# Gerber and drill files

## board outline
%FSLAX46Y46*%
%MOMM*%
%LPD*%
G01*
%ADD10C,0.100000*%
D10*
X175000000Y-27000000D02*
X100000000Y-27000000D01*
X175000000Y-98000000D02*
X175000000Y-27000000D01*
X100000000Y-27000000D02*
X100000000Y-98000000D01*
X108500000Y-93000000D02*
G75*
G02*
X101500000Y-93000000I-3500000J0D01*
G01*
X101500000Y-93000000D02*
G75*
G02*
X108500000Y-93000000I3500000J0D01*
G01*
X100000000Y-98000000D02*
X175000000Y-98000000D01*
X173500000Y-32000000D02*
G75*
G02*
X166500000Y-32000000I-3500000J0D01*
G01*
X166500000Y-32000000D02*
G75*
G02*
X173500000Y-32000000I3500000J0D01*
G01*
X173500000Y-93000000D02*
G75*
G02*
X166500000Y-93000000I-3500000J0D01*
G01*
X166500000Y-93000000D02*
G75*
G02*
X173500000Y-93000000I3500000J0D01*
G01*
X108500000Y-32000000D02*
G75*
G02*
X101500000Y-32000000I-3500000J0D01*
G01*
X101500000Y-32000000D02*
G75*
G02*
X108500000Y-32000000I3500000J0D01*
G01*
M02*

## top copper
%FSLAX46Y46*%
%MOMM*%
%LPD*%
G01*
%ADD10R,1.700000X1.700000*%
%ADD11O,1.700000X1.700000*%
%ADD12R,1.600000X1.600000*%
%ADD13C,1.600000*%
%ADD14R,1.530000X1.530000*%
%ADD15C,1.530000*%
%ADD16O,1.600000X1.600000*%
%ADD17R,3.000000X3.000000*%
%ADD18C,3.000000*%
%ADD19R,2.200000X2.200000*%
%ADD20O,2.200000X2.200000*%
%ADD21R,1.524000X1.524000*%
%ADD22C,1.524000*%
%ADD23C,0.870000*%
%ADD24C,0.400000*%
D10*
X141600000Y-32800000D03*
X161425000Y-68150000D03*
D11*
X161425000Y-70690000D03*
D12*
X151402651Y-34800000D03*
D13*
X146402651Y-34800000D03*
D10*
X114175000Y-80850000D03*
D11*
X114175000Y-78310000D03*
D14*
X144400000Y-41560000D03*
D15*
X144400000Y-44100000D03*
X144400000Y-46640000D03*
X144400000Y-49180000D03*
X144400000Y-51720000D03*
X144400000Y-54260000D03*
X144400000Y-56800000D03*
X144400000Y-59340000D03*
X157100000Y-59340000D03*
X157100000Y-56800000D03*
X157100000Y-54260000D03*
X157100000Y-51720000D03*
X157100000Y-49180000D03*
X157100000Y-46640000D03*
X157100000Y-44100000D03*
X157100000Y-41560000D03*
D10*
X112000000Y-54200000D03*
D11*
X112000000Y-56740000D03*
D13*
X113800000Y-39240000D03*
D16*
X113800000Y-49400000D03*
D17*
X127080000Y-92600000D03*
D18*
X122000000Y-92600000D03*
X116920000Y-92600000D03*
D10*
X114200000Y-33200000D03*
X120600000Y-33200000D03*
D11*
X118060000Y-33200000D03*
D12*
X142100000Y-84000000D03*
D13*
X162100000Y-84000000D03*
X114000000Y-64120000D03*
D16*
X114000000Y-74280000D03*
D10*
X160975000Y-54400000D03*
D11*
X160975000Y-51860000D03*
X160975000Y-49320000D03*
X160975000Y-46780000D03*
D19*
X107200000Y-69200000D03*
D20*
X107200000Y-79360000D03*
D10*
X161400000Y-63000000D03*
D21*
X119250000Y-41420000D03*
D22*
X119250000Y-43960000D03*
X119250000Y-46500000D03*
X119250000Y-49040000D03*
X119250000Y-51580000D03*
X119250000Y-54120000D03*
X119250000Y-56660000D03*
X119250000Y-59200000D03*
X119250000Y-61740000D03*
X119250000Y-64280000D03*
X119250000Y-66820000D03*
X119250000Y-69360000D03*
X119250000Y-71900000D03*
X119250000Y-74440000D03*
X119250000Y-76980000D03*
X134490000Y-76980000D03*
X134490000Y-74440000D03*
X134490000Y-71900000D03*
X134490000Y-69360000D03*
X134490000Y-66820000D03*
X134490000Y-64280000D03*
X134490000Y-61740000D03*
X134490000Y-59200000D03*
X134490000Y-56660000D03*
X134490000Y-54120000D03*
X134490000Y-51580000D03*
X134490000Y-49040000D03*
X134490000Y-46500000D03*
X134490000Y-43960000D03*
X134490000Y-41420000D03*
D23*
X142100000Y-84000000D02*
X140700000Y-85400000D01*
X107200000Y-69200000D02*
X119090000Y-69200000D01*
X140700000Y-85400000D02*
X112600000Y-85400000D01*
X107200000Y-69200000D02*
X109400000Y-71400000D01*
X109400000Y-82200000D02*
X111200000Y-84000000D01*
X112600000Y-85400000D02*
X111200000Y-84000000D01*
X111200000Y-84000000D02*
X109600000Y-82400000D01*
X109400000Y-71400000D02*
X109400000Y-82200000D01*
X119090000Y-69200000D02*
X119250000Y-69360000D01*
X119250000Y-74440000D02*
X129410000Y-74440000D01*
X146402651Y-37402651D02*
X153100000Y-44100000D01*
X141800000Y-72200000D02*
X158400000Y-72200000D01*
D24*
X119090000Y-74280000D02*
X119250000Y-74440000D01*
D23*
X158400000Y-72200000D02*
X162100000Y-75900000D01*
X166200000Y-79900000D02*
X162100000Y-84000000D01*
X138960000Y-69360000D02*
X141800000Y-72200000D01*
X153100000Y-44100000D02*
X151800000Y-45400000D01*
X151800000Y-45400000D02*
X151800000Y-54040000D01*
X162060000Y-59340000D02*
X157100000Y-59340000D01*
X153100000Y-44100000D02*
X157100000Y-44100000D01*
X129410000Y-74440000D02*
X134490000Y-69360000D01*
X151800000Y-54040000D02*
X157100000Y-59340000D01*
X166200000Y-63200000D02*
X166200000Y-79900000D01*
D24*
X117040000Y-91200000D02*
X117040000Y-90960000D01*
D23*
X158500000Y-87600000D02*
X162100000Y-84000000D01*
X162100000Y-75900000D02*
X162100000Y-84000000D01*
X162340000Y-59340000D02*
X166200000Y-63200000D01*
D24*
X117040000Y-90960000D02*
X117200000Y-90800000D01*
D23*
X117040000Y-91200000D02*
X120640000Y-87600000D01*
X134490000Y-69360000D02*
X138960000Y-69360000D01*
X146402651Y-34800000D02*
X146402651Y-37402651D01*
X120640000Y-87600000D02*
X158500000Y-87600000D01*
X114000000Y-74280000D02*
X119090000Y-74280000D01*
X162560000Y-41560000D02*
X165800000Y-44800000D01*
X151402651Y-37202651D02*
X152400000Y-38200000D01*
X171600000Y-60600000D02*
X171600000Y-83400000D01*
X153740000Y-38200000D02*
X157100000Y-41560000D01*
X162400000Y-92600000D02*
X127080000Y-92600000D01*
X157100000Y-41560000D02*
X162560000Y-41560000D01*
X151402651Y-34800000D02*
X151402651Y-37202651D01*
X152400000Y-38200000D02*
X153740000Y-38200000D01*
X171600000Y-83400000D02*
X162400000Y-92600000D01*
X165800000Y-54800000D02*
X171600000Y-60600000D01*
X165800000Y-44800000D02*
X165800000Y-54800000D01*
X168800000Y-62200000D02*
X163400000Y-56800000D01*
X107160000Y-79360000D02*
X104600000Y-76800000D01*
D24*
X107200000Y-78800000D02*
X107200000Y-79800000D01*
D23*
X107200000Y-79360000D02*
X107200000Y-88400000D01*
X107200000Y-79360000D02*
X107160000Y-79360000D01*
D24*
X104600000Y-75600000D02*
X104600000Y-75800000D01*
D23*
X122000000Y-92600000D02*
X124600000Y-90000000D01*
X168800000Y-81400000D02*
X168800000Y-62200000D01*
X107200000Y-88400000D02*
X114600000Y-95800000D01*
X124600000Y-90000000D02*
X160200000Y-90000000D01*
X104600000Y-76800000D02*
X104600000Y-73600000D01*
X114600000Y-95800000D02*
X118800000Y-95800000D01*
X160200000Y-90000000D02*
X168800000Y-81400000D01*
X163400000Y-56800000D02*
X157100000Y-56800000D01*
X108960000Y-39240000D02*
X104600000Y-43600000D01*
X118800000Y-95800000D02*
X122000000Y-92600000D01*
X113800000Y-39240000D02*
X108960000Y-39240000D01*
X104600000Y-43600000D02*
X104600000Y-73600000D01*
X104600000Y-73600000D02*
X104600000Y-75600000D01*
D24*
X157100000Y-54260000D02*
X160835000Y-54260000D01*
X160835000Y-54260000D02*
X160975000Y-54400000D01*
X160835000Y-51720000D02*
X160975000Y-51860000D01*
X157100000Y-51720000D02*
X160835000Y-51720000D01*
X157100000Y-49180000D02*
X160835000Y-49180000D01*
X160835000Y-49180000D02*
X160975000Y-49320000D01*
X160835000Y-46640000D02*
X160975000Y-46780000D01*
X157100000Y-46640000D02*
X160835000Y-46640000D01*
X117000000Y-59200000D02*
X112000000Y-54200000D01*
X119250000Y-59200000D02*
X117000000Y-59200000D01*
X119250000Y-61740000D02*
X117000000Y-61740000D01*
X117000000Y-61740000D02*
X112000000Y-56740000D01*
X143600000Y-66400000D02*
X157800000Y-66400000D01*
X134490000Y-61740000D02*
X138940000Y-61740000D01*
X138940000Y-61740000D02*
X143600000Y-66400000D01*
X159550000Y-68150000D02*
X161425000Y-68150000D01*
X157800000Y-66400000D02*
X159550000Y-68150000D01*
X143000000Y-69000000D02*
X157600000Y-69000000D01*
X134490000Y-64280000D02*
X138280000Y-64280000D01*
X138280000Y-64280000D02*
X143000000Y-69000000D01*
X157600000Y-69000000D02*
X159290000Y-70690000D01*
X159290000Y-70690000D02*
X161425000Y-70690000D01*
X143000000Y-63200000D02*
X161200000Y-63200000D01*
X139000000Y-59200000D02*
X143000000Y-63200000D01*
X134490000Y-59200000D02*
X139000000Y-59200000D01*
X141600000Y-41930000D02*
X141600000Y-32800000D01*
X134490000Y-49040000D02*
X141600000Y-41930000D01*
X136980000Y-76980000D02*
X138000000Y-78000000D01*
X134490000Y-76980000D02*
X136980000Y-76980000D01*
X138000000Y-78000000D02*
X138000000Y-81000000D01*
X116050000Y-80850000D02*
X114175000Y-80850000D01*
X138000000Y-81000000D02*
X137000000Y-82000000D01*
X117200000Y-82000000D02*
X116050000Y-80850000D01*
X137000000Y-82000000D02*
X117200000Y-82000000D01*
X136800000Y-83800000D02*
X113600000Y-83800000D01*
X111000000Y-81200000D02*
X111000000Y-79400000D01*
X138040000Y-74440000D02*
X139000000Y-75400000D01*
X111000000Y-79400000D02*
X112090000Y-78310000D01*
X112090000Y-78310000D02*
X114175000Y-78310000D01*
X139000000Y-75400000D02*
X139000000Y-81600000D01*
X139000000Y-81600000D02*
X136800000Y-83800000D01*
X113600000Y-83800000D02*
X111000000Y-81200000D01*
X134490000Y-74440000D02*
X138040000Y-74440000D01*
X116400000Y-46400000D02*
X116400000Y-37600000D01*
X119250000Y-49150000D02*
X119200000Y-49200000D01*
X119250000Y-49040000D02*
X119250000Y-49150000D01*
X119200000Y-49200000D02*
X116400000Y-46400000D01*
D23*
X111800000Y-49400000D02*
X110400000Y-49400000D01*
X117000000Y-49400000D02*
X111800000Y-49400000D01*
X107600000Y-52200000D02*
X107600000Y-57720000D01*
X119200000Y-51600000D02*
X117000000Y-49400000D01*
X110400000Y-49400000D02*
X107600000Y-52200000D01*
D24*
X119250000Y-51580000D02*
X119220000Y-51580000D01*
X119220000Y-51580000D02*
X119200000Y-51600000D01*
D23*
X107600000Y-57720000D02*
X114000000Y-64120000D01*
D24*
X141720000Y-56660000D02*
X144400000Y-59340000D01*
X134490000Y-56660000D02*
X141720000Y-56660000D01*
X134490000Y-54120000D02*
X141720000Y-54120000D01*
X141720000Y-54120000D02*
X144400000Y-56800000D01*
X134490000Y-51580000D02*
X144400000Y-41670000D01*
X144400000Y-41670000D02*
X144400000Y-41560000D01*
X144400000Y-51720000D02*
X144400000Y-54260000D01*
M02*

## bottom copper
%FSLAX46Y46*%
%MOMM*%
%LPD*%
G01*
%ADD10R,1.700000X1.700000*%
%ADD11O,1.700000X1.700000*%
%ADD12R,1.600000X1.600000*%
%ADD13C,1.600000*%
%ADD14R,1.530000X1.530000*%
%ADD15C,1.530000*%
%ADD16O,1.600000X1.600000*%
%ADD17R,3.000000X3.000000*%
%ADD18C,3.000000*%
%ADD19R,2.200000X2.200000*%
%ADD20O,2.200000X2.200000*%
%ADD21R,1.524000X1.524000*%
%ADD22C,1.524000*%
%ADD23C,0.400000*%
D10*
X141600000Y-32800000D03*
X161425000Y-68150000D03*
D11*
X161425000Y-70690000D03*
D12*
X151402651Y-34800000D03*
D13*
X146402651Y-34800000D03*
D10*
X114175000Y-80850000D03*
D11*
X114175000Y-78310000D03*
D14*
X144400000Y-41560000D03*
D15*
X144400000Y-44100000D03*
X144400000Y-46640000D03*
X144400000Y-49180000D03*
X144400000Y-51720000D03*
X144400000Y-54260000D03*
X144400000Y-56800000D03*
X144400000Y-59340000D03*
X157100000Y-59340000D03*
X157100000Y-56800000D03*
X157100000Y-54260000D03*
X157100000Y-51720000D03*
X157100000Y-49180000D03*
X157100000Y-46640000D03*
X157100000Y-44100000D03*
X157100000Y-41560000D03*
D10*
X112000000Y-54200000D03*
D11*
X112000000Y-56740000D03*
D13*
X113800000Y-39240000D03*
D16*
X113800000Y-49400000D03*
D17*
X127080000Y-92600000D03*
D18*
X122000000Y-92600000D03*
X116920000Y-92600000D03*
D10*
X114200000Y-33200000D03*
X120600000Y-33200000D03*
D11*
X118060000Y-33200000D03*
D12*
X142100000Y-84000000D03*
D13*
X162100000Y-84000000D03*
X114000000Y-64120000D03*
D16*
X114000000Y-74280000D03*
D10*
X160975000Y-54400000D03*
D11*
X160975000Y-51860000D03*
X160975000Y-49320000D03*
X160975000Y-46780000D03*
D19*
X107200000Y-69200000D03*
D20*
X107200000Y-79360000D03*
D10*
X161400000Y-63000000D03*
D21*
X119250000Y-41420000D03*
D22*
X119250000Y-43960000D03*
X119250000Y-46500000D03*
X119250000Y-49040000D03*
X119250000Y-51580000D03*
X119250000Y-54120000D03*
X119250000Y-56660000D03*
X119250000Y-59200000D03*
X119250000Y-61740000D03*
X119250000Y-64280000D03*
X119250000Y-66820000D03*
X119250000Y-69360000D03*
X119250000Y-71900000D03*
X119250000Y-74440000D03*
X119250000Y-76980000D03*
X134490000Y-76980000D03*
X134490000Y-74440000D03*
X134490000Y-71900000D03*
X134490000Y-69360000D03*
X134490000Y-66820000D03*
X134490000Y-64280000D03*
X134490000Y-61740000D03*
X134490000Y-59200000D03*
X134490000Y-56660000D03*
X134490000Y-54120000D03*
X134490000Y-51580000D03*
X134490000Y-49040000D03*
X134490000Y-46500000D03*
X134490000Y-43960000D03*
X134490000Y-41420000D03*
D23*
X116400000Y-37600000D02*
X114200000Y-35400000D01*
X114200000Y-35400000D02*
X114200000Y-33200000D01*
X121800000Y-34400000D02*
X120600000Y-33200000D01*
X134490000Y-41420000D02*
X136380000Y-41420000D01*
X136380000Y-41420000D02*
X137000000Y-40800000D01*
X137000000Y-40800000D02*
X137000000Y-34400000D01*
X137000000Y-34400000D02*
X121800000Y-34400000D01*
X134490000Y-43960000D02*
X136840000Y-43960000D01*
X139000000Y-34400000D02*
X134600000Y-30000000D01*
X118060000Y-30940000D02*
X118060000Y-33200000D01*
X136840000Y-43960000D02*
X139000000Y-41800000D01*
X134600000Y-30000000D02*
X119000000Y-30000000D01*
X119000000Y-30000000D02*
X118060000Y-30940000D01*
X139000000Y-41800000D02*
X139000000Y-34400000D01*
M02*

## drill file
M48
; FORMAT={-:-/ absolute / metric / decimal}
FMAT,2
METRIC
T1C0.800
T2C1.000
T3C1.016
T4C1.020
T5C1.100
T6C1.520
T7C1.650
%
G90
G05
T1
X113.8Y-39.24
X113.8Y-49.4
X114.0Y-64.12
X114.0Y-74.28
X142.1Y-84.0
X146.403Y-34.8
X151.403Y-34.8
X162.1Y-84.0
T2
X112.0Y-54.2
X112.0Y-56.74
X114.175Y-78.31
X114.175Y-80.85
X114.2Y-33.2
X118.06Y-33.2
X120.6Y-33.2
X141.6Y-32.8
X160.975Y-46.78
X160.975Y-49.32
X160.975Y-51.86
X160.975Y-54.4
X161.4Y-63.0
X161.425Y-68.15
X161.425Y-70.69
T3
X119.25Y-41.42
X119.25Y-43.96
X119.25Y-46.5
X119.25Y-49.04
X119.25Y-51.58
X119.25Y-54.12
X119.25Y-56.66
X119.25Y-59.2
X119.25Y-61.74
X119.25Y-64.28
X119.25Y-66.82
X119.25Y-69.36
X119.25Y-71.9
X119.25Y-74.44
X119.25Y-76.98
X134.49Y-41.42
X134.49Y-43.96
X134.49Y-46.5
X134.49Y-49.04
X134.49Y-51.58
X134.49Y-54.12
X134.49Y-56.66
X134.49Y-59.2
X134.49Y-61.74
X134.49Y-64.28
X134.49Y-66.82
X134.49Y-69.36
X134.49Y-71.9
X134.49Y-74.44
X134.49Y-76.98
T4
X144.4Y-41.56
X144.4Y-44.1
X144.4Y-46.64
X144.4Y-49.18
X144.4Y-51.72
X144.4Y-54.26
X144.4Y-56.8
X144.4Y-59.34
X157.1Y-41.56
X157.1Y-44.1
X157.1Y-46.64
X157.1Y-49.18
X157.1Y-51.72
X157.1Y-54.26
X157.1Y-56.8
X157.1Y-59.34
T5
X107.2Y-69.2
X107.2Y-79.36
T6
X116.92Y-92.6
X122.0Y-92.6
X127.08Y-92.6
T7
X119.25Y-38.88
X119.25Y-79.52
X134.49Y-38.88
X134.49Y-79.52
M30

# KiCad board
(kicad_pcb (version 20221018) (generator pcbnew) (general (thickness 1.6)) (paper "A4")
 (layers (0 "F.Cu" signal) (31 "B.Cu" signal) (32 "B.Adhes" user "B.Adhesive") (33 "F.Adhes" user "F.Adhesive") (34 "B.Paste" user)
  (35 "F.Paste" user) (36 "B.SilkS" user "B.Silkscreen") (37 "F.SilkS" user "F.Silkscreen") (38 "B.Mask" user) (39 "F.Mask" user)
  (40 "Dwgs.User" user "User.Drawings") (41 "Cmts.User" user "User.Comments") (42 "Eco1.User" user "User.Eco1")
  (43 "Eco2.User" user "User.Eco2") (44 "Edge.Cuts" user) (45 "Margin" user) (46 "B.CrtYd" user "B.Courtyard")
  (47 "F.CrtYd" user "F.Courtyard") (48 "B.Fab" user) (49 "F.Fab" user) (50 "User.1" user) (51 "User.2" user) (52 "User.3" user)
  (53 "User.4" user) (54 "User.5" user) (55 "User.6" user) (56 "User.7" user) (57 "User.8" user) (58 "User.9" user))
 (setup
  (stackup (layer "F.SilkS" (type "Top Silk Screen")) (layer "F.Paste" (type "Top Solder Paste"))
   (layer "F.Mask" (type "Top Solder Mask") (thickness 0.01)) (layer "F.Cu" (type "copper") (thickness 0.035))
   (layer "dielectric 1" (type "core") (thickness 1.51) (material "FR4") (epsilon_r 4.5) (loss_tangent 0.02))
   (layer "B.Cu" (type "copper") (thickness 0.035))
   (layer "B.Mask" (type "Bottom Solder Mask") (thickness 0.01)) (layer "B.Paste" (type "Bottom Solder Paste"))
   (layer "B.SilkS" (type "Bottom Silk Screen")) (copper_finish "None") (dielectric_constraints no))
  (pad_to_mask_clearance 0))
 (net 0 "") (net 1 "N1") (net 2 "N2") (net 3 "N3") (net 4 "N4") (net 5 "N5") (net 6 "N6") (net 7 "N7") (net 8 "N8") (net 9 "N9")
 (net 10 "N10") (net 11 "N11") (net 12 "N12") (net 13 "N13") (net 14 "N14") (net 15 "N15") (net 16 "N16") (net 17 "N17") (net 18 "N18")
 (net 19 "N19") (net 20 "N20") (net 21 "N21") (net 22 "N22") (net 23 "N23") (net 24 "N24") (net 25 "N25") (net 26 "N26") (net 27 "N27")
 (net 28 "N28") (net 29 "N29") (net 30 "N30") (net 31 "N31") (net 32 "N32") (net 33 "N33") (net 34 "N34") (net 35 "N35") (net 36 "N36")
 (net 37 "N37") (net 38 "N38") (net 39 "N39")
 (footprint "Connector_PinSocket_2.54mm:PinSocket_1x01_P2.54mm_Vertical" (layer "F.Cu") (at 141.6 32.8)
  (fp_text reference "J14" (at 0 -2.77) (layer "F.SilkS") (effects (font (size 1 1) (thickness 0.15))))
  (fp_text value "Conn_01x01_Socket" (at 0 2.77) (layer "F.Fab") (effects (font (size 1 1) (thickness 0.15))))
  (pad "1" thru_hole rect (at 0 0) (size 1.7 1.7) (drill 1) (layers "*.Cu" "*.Mask") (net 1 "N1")))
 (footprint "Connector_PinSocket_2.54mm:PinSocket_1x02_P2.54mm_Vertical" (layer "F.Cu") (at 161.425 68.15)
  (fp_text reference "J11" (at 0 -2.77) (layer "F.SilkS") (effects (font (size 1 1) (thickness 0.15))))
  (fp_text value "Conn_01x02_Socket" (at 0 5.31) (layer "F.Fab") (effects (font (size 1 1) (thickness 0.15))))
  (pad "1" thru_hole rect (at 0 0) (size 1.7 1.7) (drill 1) (layers "*.Cu" "*.Mask") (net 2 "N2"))
  (pad "2" thru_hole oval (at 0 2.54) (size 1.7 1.7) (drill 1) (layers "*.Cu" "*.Mask") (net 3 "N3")))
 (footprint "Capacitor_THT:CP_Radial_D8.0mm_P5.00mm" (layer "F.Cu") (at 151.402651 34.8 180)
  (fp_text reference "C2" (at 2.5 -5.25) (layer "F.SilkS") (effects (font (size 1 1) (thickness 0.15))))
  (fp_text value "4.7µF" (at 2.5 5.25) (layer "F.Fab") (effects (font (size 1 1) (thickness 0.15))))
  (pad "1" thru_hole rect (at 0 0 180) (size 1.6 1.6) (drill 0.8) (layers "*.Cu" "*.Mask") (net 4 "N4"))
  (pad "2" thru_hole circle (at 5 0 180) (size 1.6 1.6) (drill 0.8) (layers "*.Cu" "*.Mask") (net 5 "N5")))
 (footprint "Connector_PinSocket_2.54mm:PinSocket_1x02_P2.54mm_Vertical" (layer "F.Cu") (at 114.175 80.85 180)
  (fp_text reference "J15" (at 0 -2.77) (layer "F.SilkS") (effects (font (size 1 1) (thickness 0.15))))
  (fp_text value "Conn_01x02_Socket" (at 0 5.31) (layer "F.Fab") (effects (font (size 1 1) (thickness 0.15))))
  (pad "1" thru_hole rect (at 0 0 180) (size 1.7 1.7) (drill 1) (layers "*.Cu" "*.Mask") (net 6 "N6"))
  (pad "2" thru_hole oval (at 0 2.54 180) (size 1.7 1.7) (drill 1) (layers "*.Cu" "*.Mask") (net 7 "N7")))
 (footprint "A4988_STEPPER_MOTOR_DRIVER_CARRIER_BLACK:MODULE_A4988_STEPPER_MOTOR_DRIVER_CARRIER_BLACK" (layer "F.Cu") (at 150.75 50.45)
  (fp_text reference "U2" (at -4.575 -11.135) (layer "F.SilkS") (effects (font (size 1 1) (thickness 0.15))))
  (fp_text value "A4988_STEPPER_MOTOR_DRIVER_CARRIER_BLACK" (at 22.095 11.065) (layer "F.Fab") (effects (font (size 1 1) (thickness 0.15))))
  (pad "1" thru_hole rect (at -6.35 -8.89) (size 1.53 1.53) (drill 1.02) (layers "*.Cu" "*.Mask") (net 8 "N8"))
  (pad "2" thru_hole circle (at -6.35 -6.35) (size 1.53 1.53) (drill 1.02) (layers "*.Cu" "*.Mask") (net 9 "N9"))
  (pad "3" thru_hole circle (at -6.35 -3.81) (size 1.53 1.53) (drill 1.02) (layers "*.Cu" "*.Mask") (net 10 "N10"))
  (pad "4" thru_hole circle (at -6.35 -1.27) (size 1.53 1.53) (drill 1.02) (layers "*.Cu" "*.Mask") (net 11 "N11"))
  (pad "5" thru_hole circle (at -6.35 1.27) (size 1.53 1.53) (drill 1.02) (layers "*.Cu" "*.Mask") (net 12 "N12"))
  (pad "6" thru_hole circle (at -6.35 3.81) (size 1.53 1.53) (drill 1.02) (layers "*.Cu" "*.Mask") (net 12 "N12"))
  (pad "7" thru_hole circle (at -6.35 6.35) (size 1.53 1.53) (drill 1.02) (layers "*.Cu" "*.Mask") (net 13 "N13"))
  (pad "8" thru_hole circle (at -6.35 8.89) (size 1.53 1.53) (drill 1.02) (layers "*.Cu" "*.Mask") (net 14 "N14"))
  (pad "9" thru_hole circle (at 6.35 8.89) (size 1.53 1.53) (drill 1.02) (layers "*.Cu" "*.Mask") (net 5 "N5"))
  (pad "10" thru_hole circle (at 6.35 6.35) (size 1.53 1.53) (drill 1.02) (layers "*.Cu" "*.Mask") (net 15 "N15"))
  (pad "11" thru_hole circle (at 6.35 3.81) (size 1.53 1.53) (drill 1.02) (layers "*.Cu" "*.Mask") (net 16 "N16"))
  (pad "12" thru_hole circle (at 6.35 1.27) (size 1.53 1.53) (drill 1.02) (layers "*.Cu" "*.Mask") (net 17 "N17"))
  (pad "13" thru_hole circle (at 6.35 -1.27) (size 1.53 1.53) (drill 1.02) (layers "*.Cu" "*.Mask") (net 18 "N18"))
  (pad "14" thru_hole circle (at 6.35 -3.81) (size 1.53 1.53) (drill 1.02) (layers "*.Cu" "*.Mask") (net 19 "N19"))
  (pad "15" thru_hole circle (at 6.35 -6.35) (size 1.53 1.53) (drill 1.02) (layers "*.Cu" "*.Mask") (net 5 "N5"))
  (pad "16" thru_hole circle (at 6.35 -8.89) (size 1.53 1.53) (drill 1.02) (layers "*.Cu" "*.Mask") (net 4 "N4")))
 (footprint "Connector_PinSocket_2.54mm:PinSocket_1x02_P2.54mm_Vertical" (layer "F.Cu") (at 112 54.2)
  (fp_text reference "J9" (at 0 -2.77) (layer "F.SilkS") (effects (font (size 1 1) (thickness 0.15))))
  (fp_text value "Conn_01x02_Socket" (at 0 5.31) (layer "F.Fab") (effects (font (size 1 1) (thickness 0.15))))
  (pad "1" thru_hole rect (at 0 0) (size 1.7 1.7) (drill 1) (layers "*.Cu" "*.Mask") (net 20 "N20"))
  (pad "2" thru_hole oval (at 0 2.54) (size 1.7 1.7) (drill 1) (layers "*.Cu" "*.Mask") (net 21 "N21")))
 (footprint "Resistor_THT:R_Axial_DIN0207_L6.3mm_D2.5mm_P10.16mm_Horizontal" (layer "F.Cu") (at 113.8 39.24 -90)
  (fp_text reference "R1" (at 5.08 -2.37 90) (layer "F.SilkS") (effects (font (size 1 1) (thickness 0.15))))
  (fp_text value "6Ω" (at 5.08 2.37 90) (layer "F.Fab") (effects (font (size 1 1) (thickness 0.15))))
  (pad "1" thru_hole circle (at 0 0 270) (size 1.6 1.6) (drill 0.8) (layers "*.Cu" "*.Mask") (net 15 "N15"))
  (pad "2" thru_hole oval (at 10.16 0 270) (size 1.6 1.6) (drill 0.8) (layers "*.Cu" "*.Mask") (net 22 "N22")))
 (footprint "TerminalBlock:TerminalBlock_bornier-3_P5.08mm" (layer "F.Cu") (at 127.08 92.6 180)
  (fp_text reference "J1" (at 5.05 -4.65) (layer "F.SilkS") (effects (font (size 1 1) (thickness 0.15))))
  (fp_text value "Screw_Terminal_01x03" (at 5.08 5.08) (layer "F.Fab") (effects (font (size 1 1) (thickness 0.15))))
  (pad "1" thru_hole rect (at 0 0 180) (size 3 3) (drill 1.52) (layers "*.Cu" "*.Mask") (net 4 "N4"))
  (pad "2" thru_hole circle (at 5.08 0 180) (size 3 3) (drill 1.52) (layers "*.Cu" "*.Mask") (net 15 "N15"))
  (pad "3" thru_hole circle (at 10.16 0 180) (size 3 3) (drill 1.52) (layers "*.Cu" "*.Mask") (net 5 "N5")))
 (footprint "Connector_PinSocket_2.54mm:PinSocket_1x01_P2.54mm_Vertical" (layer "F.Cu") (at 114.2 33.2)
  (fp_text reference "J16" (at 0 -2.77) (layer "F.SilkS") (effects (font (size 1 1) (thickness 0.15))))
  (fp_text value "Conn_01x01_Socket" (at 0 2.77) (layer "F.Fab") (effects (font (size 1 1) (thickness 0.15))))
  (pad "1" thru_hole rect (at 0 0) (size 1.7 1.7) (drill 1) (layers "*.Cu" "*.Mask") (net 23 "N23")))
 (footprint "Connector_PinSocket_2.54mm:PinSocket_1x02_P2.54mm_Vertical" (layer "F.Cu") (at 120.6 33.2 -90)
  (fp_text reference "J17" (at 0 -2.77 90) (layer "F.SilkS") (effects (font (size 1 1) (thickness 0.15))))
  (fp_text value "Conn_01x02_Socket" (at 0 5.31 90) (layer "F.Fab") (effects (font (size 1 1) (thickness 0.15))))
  (pad "1" thru_hole rect (at 0 0 270) (size 1.7 1.7) (drill 1) (layers "*.Cu" "*.Mask") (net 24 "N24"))
  (pad "2" thru_hole oval (at 0 2.54 270) (size 1.7 1.7) (drill 1) (layers "*.Cu" "*.Mask") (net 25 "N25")))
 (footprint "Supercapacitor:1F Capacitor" (layer "F.Cu") (at 151.6 84)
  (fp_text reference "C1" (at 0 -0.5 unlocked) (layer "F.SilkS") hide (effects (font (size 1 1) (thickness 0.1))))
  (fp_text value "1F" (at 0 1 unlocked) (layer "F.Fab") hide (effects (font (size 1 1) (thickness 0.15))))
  (pad "1" thru_hole rect (at -9.5 0) (size 1.6 1.6) (drill 0.8) (layers "*.Cu" "*.Mask") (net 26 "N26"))
  (pad "2" thru_hole circle (at 10.5 0) (size 1.6 1.6) (drill 0.8) (layers "*.Cu" "*.Mask") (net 5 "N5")))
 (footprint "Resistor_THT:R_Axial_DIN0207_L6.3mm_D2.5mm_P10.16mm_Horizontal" (layer "F.Cu") (at 114 64.12 -90)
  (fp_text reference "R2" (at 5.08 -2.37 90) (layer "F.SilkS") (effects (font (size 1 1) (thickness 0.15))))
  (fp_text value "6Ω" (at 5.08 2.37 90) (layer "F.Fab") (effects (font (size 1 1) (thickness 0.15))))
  (pad "1" thru_hole circle (at 0 0 270) (size 1.6 1.6) (drill 0.8) (layers "*.Cu" "*.Mask") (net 22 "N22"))
  (pad "2" thru_hole oval (at 10.16 0 270) (size 1.6 1.6) (drill 0.8) (layers "*.Cu" "*.Mask") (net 5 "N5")))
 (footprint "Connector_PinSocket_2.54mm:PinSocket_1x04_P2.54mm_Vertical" (layer "F.Cu") (at 160.975 54.4 180)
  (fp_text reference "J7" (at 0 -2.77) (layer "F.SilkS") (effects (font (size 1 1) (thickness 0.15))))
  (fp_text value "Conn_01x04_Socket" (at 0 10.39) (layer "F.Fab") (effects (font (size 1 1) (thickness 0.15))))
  (pad "1" thru_hole rect (at 0 0 180) (size 1.7 1.7) (drill 1) (layers "*.Cu" "*.Mask") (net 16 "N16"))
  (pad "2" thru_hole oval (at 0 2.54 180) (size 1.7 1.7) (drill 1) (layers "*.Cu" "*.Mask") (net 17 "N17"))
  (pad "3" thru_hole oval (at 0 5.08 180) (size 1.7 1.7) (drill 1) (layers "*.Cu" "*.Mask") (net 18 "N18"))
  (pad "4" thru_hole oval (at 0 7.62 180) (size 1.7 1.7) (drill 1) (layers "*.Cu" "*.Mask") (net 19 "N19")))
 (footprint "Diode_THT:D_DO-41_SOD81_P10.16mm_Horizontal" (layer "F.Cu") (at 107.2 69.2 -90)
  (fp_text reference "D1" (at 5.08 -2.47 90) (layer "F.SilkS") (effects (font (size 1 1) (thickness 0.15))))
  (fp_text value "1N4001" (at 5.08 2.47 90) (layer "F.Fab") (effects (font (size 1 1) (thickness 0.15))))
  (pad "1" thru_hole rect (at 0 0 270) (size 2.2 2.2) (drill 1.1) (layers "*.Cu" "*.Mask") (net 26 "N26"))
  (pad "2" thru_hole oval (at 10.16 0 270) (size 2.2 2.2) (drill 1.1) (layers "*.Cu" "*.Mask") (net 15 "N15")))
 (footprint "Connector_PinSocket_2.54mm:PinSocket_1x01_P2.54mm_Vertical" (layer "F.Cu") (at 161.4 63)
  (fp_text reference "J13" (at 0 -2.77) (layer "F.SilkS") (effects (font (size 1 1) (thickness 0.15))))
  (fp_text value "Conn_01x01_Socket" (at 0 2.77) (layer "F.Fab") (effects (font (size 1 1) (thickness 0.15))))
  (pad "1" thru_hole rect (at 0 0) (size 1.7 1.7) (drill 1) (layers "*.Cu" "*.Mask") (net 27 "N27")))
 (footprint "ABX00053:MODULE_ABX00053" (layer "F.Cu") (at 126.87 59.2 -90)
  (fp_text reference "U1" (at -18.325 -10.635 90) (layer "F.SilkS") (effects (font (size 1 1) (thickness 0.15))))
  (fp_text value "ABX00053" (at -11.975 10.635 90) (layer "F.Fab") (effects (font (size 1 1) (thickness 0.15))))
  (pad "" np_thru_hole circle (at -20.32 -7.62 270) (size 1.65 1.65) (drill 1.65) (layers "*.Cu" "*.Mask"))
  (pad "" np_thru_hole circle (at -20.32 7.62 270) (size 1.65 1.65) (drill 1.65) (layers "*.Cu" "*.Mask"))
  (pad "" np_thru_hole circle (at 20.32 -7.62 270) (size 1.65 1.65) (drill 1.65) (layers "*.Cu" "*.Mask"))
  (pad "" np_thru_hole circle (at 20.32 7.62 270) (size 1.65 1.65) (drill 1.65) (layers "*.Cu" "*.Mask"))
  (pad "1" thru_hole rect (at -17.78 7.62 270) (size 1.524 1.524) (drill 1.016) (layers "*.Cu" "*.Mask") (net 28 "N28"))
  (pad "2" thru_hole circle (at -15.24 7.62 270) (size 1.524 1.524) (drill 1.016) (layers "*.Cu" "*.Mask") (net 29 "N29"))
  (pad "3" thru_hole circle (at -12.7 7.62 270) (size 1.524 1.524) (drill 1.016) (layers "*.Cu" "*.Mask") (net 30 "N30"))
  (pad "4" thru_hole circle (at -10.16 7.62 270) (size 1.524 1.524) (drill 1.016) (layers "*.Cu" "*.Mask") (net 23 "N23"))
  (pad "5" thru_hole circle (at -7.62 7.62 270) (size 1.524 1.524) (drill 1.016) (layers "*.Cu" "*.Mask") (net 22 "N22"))
  (pad "6" thru_hole circle (at -5.08 7.62 270) (size 1.524 1.524) (drill 1.016) (layers "*.Cu" "*.Mask") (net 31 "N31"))
  (pad "7" thru_hole circle (at -2.54 7.62 270) (size 1.524 1.524) (drill 1.016) (layers "*.Cu" "*.Mask") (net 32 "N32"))
  (pad "8" thru_hole circle (at 0 7.62 270) (size 1.524 1.524) (drill 1.016) (layers "*.Cu" "*.Mask") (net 20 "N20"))
  (pad "9" thru_hole circle (at 2.54 7.62 270) (size 1.524 1.524) (drill 1.016) (layers "*.Cu" "*.Mask") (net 21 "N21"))
  (pad "10" thru_hole circle (at 5.08 7.62 270) (size 1.524 1.524) (drill 1.016) (layers "*.Cu" "*.Mask") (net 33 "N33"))
  (pad "11" thru_hole circle (at 7.62 7.62 270) (size 1.524 1.524) (drill 1.016) (layers "*.Cu" "*.Mask") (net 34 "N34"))
  (pad "12" thru_hole circle (at 10.16 7.62 270) (size 1.524 1.524) (drill 1.016) (layers "*.Cu" "*.Mask") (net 26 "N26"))
  (pad "13" thru_hole circle (at 12.7 7.62 270) (size 1.524 1.524) (drill 1.016) (layers "*.Cu" "*.Mask") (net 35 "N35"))
  (pad "14" thru_hole circle (at 15.24 7.62 270) (size 1.524 1.524) (drill 1.016) (layers "*.Cu" "*.Mask") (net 5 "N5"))
  (pad "15" thru_hole circle (at 17.78 7.62 270) (size 1.524 1.524) (drill 1.016) (layers "*.Cu" "*.Mask") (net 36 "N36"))
  (pad "16" thru_hole circle (at 17.78 -7.62 270) (size 1.524 1.524) (drill 1.016) (layers "*.Cu" "*.Mask") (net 6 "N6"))
  (pad "17" thru_hole circle (at 15.24 -7.62 270) (size 1.524 1.524) (drill 1.016) (layers "*.Cu" "*.Mask") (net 7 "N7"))
  (pad "18" thru_hole circle (at 12.7 -7.62 270) (size 1.524 1.524) (drill 1.016) (layers "*.Cu" "*.Mask") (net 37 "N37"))
  (pad "19" thru_hole circle (at 10.16 -7.62 270) (size 1.524 1.524) (drill 1.016) (layers "*.Cu" "*.Mask") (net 5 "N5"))
  (pad "20" thru_hole circle (at 7.62 -7.62 270) (size 1.524 1.524) (drill 1.016) (layers "*.Cu" "*.Mask") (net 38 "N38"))
  (pad "21" thru_hole circle (at 5.08 -7.62 270) (size 1.524 1.524) (drill 1.016) (layers "*.Cu" "*.Mask") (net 3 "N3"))
  (pad "22" thru_hole circle (at 2.54 -7.62 270) (size 1.524 1.524) (drill 1.016) (layers "*.Cu" "*.Mask") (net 2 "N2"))
  (pad "23" thru_hole circle (at 0 -7.62 270) (size 1.524 1.524) (drill 1.016) (layers "*.Cu" "*.Mask") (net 27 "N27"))
  (pad "24" thru_hole circle (at -2.54 -7.62 270) (size 1.524 1.524) (drill 1.016) (layers "*.Cu" "*.Mask") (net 14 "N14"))
  (pad "25" thru_hole circle (at -5.08 -7.62 270) (size 1.524 1.524) (drill 1.016) (layers "*.Cu" "*.Mask") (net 13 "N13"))
  (pad "26" thru_hole circle (at -7.62 -7.62 270) (size 1.524 1.524) (drill 1.016) (layers "*.Cu" "*.Mask") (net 8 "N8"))
  (pad "27" thru_hole circle (at -10.16 -7.62 270) (size 1.524 1.524) (drill 1.016) (layers "*.Cu" "*.Mask") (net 1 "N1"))
  (pad "28" thru_hole circle (at -12.7 -7.62 270) (size 1.524 1.524) (drill 1.016) (layers "*.Cu" "*.Mask") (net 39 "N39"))
  (pad "29" thru_hole circle (at -15.24 -7.62 270) (size 1.524 1.524) (drill 1.016) (layers "*.Cu" "*.Mask") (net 25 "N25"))
  (pad "30" thru_hole circle (at -17.78 -7.62 270) (size 1.524 1.524) (drill 1.016) (layers "*.Cu" "*.Mask") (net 24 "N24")))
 (gr_line (start 175 27) (end 100 27) (stroke (width 0.1) (type default)) (layer "Edge.Cuts"))
 (gr_line (start 175 98) (end 175 27) (stroke (width 0.1) (type default)) (layer "Edge.Cuts"))
 (gr_line (start 100 27) (end 100 98) (stroke (width 0.1) (type default)) (layer "Edge.Cuts"))
 (gr_circle (center 105 93) (end 108.5 93) (stroke (width 0.1) (type default)) (fill none) (layer "Edge.Cuts"))
 (gr_line (start 100 98) (end 175 98) (stroke (width 0.1) (type default)) (layer "Edge.Cuts"))
 (gr_circle (center 170 32) (end 173.5 32) (stroke (width 0.1) (type default)) (fill none) (layer "Edge.Cuts"))
 (gr_circle (center 170 93) (end 173.5 93) (stroke (width 0.1) (type default)) (fill none) (layer "Edge.Cuts"))
 (gr_circle (center 105 32) (end 108.5 32) (stroke (width 0.1) (type default)) (fill none) (layer "Edge.Cuts"))
 (segment (start 142.1 84) (end 140.7 85.4) (width 0.87) (layer "F.Cu") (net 26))
 (segment (start 107.2 69.2) (end 119.09 69.2) (width 0.87) (layer "F.Cu") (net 26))
 (segment (start 140.7 85.4) (end 112.6 85.4) (width 0.87) (layer "F.Cu") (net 26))
 (segment (start 107.2 69.2) (end 109.4 71.4) (width 0.87) (layer "F.Cu") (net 26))
 (segment (start 109.4 82.2) (end 111.2 84) (width 0.87) (layer "F.Cu") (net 26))
 (segment (start 112.6 85.4) (end 111.2 84) (width 0.87) (layer "F.Cu") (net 26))
 (segment (start 111.2 84) (end 109.6 82.4) (width 0.87) (layer "F.Cu") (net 26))
 (segment (start 109.4 71.4) (end 109.4 82.2) (width 0.87) (layer "F.Cu") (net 26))
 (segment (start 119.09 69.2) (end 119.25 69.36) (width 0.87) (layer "F.Cu") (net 26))
 (segment (start 119.25 74.44) (end 129.41 74.44) (width 0.87) (layer "F.Cu") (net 5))
 (segment (start 146.402651 37.402651) (end 153.1 44.1) (width 0.87) (layer "F.Cu") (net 5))
 (segment (start 141.8 72.2) (end 158.4 72.2) (width 0.87) (layer "F.Cu") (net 5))
 (segment (start 119.09 74.28) (end 119.25 74.44) (width 0.4) (layer "F.Cu") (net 5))
 (segment (start 158.4 72.2) (end 162.1 75.9) (width 0.87) (layer "F.Cu") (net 5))
 (segment (start 166.2 79.9) (end 162.1 84) (width 0.87) (layer "F.Cu") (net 5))
 (segment (start 138.96 69.36) (end 141.8 72.2) (width 0.87) (layer "F.Cu") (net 5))
 (segment (start 153.1 44.1) (end 151.8 45.4) (width 0.87) (layer "F.Cu") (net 5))
 (segment (start 151.8 45.4) (end 151.8 54.04) (width 0.87) (layer "F.Cu") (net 5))
 (segment (start 162.06 59.34) (end 157.1 59.34) (width 0.87) (layer "F.Cu") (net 5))
 (segment (start 153.1 44.1) (end 157.1 44.1) (width 0.87) (layer "F.Cu") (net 5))
 (segment (start 129.41 74.44) (end 134.49 69.36) (width 0.87) (layer "F.Cu") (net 5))
 (segment (start 151.8 54.04) (end 157.1 59.34) (width 0.87) (layer "F.Cu") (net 5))
 (segment (start 166.2 63.2) (end 166.2 79.9) (width 0.87) (layer "F.Cu") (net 5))
 (segment (start 117.04 91.2) (end 117.04 90.96) (width 0.4) (layer "F.Cu") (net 5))
 (segment (start 158.5 87.6) (end 162.1 84) (width 0.87) (layer "F.Cu") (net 5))
 (segment (start 162.1 75.9) (end 162.1 84) (width 0.87) (layer "F.Cu") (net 5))
 (segment (start 162.34 59.34) (end 166.2 63.2) (width 0.87) (layer "F.Cu") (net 5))
 (segment (start 117.04 90.96) (end 117.2 90.8) (width 0.4) (layer "F.Cu") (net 5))
 (segment (start 117.04 91.2) (end 120.64 87.6) (width 0.87) (layer "F.Cu") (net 5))
 (segment (start 134.49 69.36) (end 138.96 69.36) (width 0.87) (layer "F.Cu") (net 5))
 (segment (start 146.402651 34.8) (end 146.402651 37.402651) (width 0.87) (layer "F.Cu") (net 5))
 (segment (start 120.64 87.6) (end 158.5 87.6) (width 0.87) (layer "F.Cu") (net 5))
 (segment (start 114 74.28) (end 119.09 74.28) (width 0.87) (layer "F.Cu") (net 5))
 (segment (start 162.56 41.56) (end 165.8 44.8) (width 0.87) (layer "F.Cu") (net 4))
 (segment (start 151.402651 37.202651) (end 152.4 38.2) (width 0.87) (layer "F.Cu") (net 4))
 (segment (start 171.6 60.6) (end 171.6 83.4) (width 0.87) (layer "F.Cu") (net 4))
 (segment (start 153.74 38.2) (end 157.1 41.56) (width 0.87) (layer "F.Cu") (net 4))
 (segment (start 162.4 92.6) (end 127.08 92.6) (width 0.87) (layer "F.Cu") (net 4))
 (segment (start 157.1 41.56) (end 162.56 41.56) (width 0.87) (layer "F.Cu") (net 4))
 (segment (start 151.402651 34.8) (end 151.402651 37.202651) (width 0.87) (layer "F.Cu") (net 4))
 (segment (start 152.4 38.2) (end 153.74 38.2) (width 0.87) (layer "F.Cu") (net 4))
 (segment (start 171.6 83.4) (end 162.4 92.6) (width 0.87) (layer "F.Cu") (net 4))
 (segment (start 165.8 54.8) (end 171.6 60.6) (width 0.87) (layer "F.Cu") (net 4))
 (segment (start 165.8 44.8) (end 165.8 54.8) (width 0.87) (layer "F.Cu") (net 4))
 (segment (start 168.8 62.2) (end 163.4 56.8) (width 0.87) (layer "F.Cu") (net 15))
 (segment (start 107.16 79.36) (end 104.6 76.8) (width 0.87) (layer "F.Cu") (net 15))
 (segment (start 107.2 78.8) (end 107.2 79.8) (width 0.4) (layer "F.Cu") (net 15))
 (segment (start 107.2 79.36) (end 107.2 88.4) (width 0.87) (layer "F.Cu") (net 15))
 (segment (start 107.2 79.36) (end 107.16 79.36) (width 0.87) (layer "F.Cu") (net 15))
 (segment (start 104.6 75.6) (end 104.6 75.8) (width 0.4) (layer "F.Cu") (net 15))
 (segment (start 122 92.6) (end 124.6 90) (width 0.87) (layer "F.Cu") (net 15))
 (segment (start 168.8 81.4) (end 168.8 62.2) (width 0.87) (layer "F.Cu") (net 15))
 (segment (start 107.2 88.4) (end 114.6 95.8) (width 0.87) (layer "F.Cu") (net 15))
 (segment (start 124.6 90) (end 160.2 90) (width 0.87) (layer "F.Cu") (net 15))
 (segment (start 104.6 76.8) (end 104.6 73.6) (width 0.87) (layer "F.Cu") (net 15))
 (segment (start 114.6 95.8) (end 118.8 95.8) (width 0.87) (layer "F.Cu") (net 15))
 (segment (start 160.2 90) (end 168.8 81.4) (width 0.87) (layer "F.Cu") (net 15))
 (segment (start 163.4 56.8) (end 157.1 56.8) (width 0.87) (layer "F.Cu") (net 15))
 (segment (start 108.96 39.24) (end 104.6 43.6) (width 0.87) (layer "F.Cu") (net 15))
 (segment (start 118.8 95.8) (end 122 92.6) (width 0.87) (layer "F.Cu") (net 15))
 (segment (start 113.8 39.24) (end 108.96 39.24) (width 0.87) (layer "F.Cu") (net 15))
 (segment (start 104.6 43.6) (end 104.6 73.6) (width 0.87) (layer "F.Cu") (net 15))
 (segment (start 104.6 73.6) (end 104.6 75.6) (width 0.87) (layer "F.Cu") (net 15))
 (segment (start 157.1 54.26) (end 160.835 54.26) (width 0.4) (layer "F.Cu") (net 16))
 (segment (start 160.835 54.26) (end 160.975 54.4) (width 0.4) (layer "F.Cu") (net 16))
 (segment (start 160.835 51.72) (end 160.975 51.86) (width 0.4) (layer "F.Cu") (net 17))
 (segment (start 157.1 51.72) (end 160.835 51.72) (width 0.4) (layer "F.Cu") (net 17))
 (segment (start 157.1 49.18) (end 160.835 49.18) (width 0.4) (layer "F.Cu") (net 18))
 (segment (start 160.835 49.18) (end 160.975 49.32) (width 0.4) (layer "F.Cu") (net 18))
 (segment (start 160.835 46.64) (end 160.975 46.78) (width 0.4) (layer "F.Cu") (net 19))
 (segment (start 157.1 46.64) (end 160.835 46.64) (width 0.4) (layer "F.Cu") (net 19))
 (segment (start 117 59.2) (end 112 54.2) (width 0.4) (layer "F.Cu") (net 20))
 (segment (start 119.25 59.2) (end 117 59.2) (width 0.4) (layer "F.Cu") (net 20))
 (segment (start 119.25 61.74) (end 117 61.74) (width 0.4) (layer "F.Cu") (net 21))
 (segment (start 117 61.74) (end 112 56.74) (width 0.4) (layer "F.Cu") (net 21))
 (segment (start 143.6 66.4) (end 157.8 66.4) (width 0.4) (layer "F.Cu") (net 2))
 (segment (start 134.49 61.74) (end 138.94 61.74) (width 0.4) (layer "F.Cu") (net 2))
 (segment (start 138.94 61.74) (end 143.6 66.4) (width 0.4) (layer "F.Cu") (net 2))
 (segment (start 159.55 68.15) (end 161.425 68.15) (width 0.4) (layer "F.Cu") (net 2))
 (segment (start 157.8 66.4) (end 159.55 68.15) (width 0.4) (layer "F.Cu") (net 2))
 (segment (start 143 69) (end 157.6 69) (width 0.4) (layer "F.Cu") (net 3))
 (segment (start 134.49 64.28) (end 138.28 64.28) (width 0.4) (layer "F.Cu") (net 3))
 (segment (start 138.28 64.28) (end 143 69) (width 0.4) (layer "F.Cu") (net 3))
 (segment (start 157.6 69) (end 159.29 70.69) (width 0.4) (layer "F.Cu") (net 3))
 (segment (start 159.29 70.69) (end 161.425 70.69) (width 0.4) (layer "F.Cu") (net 3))
 (segment (start 143 63.2) (end 161.2 63.2) (width 0.4) (layer "F.Cu") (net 27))
 (segment (start 139 59.2) (end 143 63.2) (width 0.4) (layer "F.Cu") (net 27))
 (segment (start 134.49 59.2) (end 139 59.2) (width 0.4) (layer "F.Cu") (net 27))
 (segment (start 141.6 41.93) (end 141.6 32.8) (width 0.4) (layer "F.Cu") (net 1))
 (segment (start 134.49 49.04) (end 141.6 41.93) (width 0.4) (layer "F.Cu") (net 1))
 (segment (start 136.98 76.98) (end 138 78) (width 0.4) (layer "F.Cu") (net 6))
 (segment (start 134.49 76.98) (end 136.98 76.98) (width 0.4) (layer "F.Cu") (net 6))
 (segment (start 138 78) (end 138 81) (width 0.4) (layer "F.Cu") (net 6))
 (segment (start 116.05 80.85) (end 114.175 80.85) (width 0.4) (layer "F.Cu") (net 6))
 (segment (start 138 81) (end 137 82) (width 0.4) (layer "F.Cu") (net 6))
 (segment (start 117.2 82) (end 116.05 80.85) (width 0.4) (layer "F.Cu") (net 6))
 (segment (start 137 82) (end 117.2 82) (width 0.4) (layer "F.Cu") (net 6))
 (segment (start 136.8 83.8) (end 113.6 83.8) (width 0.4) (layer "F.Cu") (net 7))
 (segment (start 111 81.2) (end 111 79.4) (width 0.4) (layer "F.Cu") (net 7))
 (segment (start 138.04 74.44) (end 139 75.4) (width 0.4) (layer "F.Cu") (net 7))
 (segment (start 111 79.4) (end 112.09 78.31) (width 0.4) (layer "F.Cu") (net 7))
 (segment (start 112.09 78.31) (end 114.175 78.31) (width 0.4) (layer "F.Cu") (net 7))
 (segment (start 139 75.4) (end 139 81.6) (width 0.4) (layer "F.Cu") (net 7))
 (segment (start 139 81.6) (end 136.8 83.8) (width 0.4) (layer "F.Cu") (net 7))
 (segment (start 113.6 83.8) (end 111 81.2) (width 0.4) (layer "F.Cu") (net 7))
 (segment (start 134.49 74.44) (end 138.04 74.44) (width 0.4) (layer "F.Cu") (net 7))
 (segment (start 116.4 46.4) (end 116.4 37.6) (width 0.4) (layer "F.Cu") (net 23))
 (segment (start 119.25 49.15) (end 119.2 49.2) (width 0.4) (layer "F.Cu") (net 23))
 (segment (start 119.25 49.04) (end 119.25 49.15) (width 0.4) (layer "F.Cu") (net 23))
 (segment (start 119.2 49.2) (end 116.4 46.4) (width 0.4) (layer "F.Cu") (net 23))
 (segment (start 116.4 37.6) (end 114.2 35.4) (width 0.4) (layer "B.Cu") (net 23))
 (segment (start 114.2 35.4) (end 114.2 33.2) (width 0.4) (layer "B.Cu") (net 23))
 (segment (start 121.8 34.4) (end 120.6 33.2) (width 0.4) (layer "B.Cu") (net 24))
 (segment (start 134.49 41.42) (end 136.38 41.42) (width 0.4) (layer "B.Cu") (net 24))
 (segment (start 136.38 41.42) (end 137 40.8) (width 0.4) (layer "B.Cu") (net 24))
 (segment (start 137 40.8) (end 137 34.4) (width 0.4) (layer "B.Cu") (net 24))
 (segment (start 137 34.4) (end 121.8 34.4) (width 0.4) (layer "B.Cu") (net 24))
 (segment (start 134.49 43.96) (end 136.84 43.96) (width 0.4) (layer "B.Cu") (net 25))
 (segment (start 139 34.4) (end 134.6 30) (width 0.4) (layer "B.Cu") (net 25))
 (segment (start 118.06 30.94) (end 118.06 33.2) (width 0.4) (layer "B.Cu") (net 25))
 (segment (start 136.84 43.96) (end 139 41.8) (width 0.4) (layer "B.Cu") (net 25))
 (segment (start 134.6 30) (end 119 30) (width 0.4) (layer "B.Cu") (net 25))
 (segment (start 119 30) (end 118.06 30.94) (width 0.4) (layer "B.Cu") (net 25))
 (segment (start 139 41.8) (end 139 34.4) (width 0.4) (layer "B.Cu") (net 25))
 (segment (start 111.8 49.4) (end 110.4 49.4) (width 0.87) (layer "F.Cu") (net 22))
 (segment (start 117 49.4) (end 111.8 49.4) (width 0.87) (layer "F.Cu") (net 22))
 (segment (start 107.6 52.2) (end 107.6 57.72) (width 0.87) (layer "F.Cu") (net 22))
 (segment (start 119.2 51.6) (end 117 49.4) (width 0.87) (layer "F.Cu") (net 22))
 (segment (start 110.4 49.4) (end 107.6 52.2) (width 0.87) (layer "F.Cu") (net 22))
 (segment (start 119.25 51.58) (end 119.22 51.58) (width 0.4) (layer "F.Cu") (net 22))
 (segment (start 119.22 51.58) (end 119.2 51.6) (width 0.4) (layer "F.Cu") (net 22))
 (segment (start 107.6 57.72) (end 114 64.12) (width 0.87) (layer "F.Cu") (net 22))
 (segment (start 141.72 56.66) (end 144.4 59.34) (width 0.4) (layer "F.Cu") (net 14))
 (segment (start 134.49 56.66) (end 141.72 56.66) (width 0.4) (layer "F.Cu") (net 14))
 (segment (start 134.49 54.12) (end 141.72 54.12) (width 0.4) (layer "F.Cu") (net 13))
 (segment (start 141.72 54.12) (end 144.4 56.8) (width 0.4) (layer "F.Cu") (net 13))
 (segment (start 134.49 51.58) (end 144.4 41.67) (width 0.4) (layer "F.Cu") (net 8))
 (segment (start 144.4 41.67) (end 144.4 41.56) (width 0.4) (layer "F.Cu") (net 8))
 (segment (start 144.4 51.72) (end 144.4 54.26) (width 0.4) (layer "F.Cu") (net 12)))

